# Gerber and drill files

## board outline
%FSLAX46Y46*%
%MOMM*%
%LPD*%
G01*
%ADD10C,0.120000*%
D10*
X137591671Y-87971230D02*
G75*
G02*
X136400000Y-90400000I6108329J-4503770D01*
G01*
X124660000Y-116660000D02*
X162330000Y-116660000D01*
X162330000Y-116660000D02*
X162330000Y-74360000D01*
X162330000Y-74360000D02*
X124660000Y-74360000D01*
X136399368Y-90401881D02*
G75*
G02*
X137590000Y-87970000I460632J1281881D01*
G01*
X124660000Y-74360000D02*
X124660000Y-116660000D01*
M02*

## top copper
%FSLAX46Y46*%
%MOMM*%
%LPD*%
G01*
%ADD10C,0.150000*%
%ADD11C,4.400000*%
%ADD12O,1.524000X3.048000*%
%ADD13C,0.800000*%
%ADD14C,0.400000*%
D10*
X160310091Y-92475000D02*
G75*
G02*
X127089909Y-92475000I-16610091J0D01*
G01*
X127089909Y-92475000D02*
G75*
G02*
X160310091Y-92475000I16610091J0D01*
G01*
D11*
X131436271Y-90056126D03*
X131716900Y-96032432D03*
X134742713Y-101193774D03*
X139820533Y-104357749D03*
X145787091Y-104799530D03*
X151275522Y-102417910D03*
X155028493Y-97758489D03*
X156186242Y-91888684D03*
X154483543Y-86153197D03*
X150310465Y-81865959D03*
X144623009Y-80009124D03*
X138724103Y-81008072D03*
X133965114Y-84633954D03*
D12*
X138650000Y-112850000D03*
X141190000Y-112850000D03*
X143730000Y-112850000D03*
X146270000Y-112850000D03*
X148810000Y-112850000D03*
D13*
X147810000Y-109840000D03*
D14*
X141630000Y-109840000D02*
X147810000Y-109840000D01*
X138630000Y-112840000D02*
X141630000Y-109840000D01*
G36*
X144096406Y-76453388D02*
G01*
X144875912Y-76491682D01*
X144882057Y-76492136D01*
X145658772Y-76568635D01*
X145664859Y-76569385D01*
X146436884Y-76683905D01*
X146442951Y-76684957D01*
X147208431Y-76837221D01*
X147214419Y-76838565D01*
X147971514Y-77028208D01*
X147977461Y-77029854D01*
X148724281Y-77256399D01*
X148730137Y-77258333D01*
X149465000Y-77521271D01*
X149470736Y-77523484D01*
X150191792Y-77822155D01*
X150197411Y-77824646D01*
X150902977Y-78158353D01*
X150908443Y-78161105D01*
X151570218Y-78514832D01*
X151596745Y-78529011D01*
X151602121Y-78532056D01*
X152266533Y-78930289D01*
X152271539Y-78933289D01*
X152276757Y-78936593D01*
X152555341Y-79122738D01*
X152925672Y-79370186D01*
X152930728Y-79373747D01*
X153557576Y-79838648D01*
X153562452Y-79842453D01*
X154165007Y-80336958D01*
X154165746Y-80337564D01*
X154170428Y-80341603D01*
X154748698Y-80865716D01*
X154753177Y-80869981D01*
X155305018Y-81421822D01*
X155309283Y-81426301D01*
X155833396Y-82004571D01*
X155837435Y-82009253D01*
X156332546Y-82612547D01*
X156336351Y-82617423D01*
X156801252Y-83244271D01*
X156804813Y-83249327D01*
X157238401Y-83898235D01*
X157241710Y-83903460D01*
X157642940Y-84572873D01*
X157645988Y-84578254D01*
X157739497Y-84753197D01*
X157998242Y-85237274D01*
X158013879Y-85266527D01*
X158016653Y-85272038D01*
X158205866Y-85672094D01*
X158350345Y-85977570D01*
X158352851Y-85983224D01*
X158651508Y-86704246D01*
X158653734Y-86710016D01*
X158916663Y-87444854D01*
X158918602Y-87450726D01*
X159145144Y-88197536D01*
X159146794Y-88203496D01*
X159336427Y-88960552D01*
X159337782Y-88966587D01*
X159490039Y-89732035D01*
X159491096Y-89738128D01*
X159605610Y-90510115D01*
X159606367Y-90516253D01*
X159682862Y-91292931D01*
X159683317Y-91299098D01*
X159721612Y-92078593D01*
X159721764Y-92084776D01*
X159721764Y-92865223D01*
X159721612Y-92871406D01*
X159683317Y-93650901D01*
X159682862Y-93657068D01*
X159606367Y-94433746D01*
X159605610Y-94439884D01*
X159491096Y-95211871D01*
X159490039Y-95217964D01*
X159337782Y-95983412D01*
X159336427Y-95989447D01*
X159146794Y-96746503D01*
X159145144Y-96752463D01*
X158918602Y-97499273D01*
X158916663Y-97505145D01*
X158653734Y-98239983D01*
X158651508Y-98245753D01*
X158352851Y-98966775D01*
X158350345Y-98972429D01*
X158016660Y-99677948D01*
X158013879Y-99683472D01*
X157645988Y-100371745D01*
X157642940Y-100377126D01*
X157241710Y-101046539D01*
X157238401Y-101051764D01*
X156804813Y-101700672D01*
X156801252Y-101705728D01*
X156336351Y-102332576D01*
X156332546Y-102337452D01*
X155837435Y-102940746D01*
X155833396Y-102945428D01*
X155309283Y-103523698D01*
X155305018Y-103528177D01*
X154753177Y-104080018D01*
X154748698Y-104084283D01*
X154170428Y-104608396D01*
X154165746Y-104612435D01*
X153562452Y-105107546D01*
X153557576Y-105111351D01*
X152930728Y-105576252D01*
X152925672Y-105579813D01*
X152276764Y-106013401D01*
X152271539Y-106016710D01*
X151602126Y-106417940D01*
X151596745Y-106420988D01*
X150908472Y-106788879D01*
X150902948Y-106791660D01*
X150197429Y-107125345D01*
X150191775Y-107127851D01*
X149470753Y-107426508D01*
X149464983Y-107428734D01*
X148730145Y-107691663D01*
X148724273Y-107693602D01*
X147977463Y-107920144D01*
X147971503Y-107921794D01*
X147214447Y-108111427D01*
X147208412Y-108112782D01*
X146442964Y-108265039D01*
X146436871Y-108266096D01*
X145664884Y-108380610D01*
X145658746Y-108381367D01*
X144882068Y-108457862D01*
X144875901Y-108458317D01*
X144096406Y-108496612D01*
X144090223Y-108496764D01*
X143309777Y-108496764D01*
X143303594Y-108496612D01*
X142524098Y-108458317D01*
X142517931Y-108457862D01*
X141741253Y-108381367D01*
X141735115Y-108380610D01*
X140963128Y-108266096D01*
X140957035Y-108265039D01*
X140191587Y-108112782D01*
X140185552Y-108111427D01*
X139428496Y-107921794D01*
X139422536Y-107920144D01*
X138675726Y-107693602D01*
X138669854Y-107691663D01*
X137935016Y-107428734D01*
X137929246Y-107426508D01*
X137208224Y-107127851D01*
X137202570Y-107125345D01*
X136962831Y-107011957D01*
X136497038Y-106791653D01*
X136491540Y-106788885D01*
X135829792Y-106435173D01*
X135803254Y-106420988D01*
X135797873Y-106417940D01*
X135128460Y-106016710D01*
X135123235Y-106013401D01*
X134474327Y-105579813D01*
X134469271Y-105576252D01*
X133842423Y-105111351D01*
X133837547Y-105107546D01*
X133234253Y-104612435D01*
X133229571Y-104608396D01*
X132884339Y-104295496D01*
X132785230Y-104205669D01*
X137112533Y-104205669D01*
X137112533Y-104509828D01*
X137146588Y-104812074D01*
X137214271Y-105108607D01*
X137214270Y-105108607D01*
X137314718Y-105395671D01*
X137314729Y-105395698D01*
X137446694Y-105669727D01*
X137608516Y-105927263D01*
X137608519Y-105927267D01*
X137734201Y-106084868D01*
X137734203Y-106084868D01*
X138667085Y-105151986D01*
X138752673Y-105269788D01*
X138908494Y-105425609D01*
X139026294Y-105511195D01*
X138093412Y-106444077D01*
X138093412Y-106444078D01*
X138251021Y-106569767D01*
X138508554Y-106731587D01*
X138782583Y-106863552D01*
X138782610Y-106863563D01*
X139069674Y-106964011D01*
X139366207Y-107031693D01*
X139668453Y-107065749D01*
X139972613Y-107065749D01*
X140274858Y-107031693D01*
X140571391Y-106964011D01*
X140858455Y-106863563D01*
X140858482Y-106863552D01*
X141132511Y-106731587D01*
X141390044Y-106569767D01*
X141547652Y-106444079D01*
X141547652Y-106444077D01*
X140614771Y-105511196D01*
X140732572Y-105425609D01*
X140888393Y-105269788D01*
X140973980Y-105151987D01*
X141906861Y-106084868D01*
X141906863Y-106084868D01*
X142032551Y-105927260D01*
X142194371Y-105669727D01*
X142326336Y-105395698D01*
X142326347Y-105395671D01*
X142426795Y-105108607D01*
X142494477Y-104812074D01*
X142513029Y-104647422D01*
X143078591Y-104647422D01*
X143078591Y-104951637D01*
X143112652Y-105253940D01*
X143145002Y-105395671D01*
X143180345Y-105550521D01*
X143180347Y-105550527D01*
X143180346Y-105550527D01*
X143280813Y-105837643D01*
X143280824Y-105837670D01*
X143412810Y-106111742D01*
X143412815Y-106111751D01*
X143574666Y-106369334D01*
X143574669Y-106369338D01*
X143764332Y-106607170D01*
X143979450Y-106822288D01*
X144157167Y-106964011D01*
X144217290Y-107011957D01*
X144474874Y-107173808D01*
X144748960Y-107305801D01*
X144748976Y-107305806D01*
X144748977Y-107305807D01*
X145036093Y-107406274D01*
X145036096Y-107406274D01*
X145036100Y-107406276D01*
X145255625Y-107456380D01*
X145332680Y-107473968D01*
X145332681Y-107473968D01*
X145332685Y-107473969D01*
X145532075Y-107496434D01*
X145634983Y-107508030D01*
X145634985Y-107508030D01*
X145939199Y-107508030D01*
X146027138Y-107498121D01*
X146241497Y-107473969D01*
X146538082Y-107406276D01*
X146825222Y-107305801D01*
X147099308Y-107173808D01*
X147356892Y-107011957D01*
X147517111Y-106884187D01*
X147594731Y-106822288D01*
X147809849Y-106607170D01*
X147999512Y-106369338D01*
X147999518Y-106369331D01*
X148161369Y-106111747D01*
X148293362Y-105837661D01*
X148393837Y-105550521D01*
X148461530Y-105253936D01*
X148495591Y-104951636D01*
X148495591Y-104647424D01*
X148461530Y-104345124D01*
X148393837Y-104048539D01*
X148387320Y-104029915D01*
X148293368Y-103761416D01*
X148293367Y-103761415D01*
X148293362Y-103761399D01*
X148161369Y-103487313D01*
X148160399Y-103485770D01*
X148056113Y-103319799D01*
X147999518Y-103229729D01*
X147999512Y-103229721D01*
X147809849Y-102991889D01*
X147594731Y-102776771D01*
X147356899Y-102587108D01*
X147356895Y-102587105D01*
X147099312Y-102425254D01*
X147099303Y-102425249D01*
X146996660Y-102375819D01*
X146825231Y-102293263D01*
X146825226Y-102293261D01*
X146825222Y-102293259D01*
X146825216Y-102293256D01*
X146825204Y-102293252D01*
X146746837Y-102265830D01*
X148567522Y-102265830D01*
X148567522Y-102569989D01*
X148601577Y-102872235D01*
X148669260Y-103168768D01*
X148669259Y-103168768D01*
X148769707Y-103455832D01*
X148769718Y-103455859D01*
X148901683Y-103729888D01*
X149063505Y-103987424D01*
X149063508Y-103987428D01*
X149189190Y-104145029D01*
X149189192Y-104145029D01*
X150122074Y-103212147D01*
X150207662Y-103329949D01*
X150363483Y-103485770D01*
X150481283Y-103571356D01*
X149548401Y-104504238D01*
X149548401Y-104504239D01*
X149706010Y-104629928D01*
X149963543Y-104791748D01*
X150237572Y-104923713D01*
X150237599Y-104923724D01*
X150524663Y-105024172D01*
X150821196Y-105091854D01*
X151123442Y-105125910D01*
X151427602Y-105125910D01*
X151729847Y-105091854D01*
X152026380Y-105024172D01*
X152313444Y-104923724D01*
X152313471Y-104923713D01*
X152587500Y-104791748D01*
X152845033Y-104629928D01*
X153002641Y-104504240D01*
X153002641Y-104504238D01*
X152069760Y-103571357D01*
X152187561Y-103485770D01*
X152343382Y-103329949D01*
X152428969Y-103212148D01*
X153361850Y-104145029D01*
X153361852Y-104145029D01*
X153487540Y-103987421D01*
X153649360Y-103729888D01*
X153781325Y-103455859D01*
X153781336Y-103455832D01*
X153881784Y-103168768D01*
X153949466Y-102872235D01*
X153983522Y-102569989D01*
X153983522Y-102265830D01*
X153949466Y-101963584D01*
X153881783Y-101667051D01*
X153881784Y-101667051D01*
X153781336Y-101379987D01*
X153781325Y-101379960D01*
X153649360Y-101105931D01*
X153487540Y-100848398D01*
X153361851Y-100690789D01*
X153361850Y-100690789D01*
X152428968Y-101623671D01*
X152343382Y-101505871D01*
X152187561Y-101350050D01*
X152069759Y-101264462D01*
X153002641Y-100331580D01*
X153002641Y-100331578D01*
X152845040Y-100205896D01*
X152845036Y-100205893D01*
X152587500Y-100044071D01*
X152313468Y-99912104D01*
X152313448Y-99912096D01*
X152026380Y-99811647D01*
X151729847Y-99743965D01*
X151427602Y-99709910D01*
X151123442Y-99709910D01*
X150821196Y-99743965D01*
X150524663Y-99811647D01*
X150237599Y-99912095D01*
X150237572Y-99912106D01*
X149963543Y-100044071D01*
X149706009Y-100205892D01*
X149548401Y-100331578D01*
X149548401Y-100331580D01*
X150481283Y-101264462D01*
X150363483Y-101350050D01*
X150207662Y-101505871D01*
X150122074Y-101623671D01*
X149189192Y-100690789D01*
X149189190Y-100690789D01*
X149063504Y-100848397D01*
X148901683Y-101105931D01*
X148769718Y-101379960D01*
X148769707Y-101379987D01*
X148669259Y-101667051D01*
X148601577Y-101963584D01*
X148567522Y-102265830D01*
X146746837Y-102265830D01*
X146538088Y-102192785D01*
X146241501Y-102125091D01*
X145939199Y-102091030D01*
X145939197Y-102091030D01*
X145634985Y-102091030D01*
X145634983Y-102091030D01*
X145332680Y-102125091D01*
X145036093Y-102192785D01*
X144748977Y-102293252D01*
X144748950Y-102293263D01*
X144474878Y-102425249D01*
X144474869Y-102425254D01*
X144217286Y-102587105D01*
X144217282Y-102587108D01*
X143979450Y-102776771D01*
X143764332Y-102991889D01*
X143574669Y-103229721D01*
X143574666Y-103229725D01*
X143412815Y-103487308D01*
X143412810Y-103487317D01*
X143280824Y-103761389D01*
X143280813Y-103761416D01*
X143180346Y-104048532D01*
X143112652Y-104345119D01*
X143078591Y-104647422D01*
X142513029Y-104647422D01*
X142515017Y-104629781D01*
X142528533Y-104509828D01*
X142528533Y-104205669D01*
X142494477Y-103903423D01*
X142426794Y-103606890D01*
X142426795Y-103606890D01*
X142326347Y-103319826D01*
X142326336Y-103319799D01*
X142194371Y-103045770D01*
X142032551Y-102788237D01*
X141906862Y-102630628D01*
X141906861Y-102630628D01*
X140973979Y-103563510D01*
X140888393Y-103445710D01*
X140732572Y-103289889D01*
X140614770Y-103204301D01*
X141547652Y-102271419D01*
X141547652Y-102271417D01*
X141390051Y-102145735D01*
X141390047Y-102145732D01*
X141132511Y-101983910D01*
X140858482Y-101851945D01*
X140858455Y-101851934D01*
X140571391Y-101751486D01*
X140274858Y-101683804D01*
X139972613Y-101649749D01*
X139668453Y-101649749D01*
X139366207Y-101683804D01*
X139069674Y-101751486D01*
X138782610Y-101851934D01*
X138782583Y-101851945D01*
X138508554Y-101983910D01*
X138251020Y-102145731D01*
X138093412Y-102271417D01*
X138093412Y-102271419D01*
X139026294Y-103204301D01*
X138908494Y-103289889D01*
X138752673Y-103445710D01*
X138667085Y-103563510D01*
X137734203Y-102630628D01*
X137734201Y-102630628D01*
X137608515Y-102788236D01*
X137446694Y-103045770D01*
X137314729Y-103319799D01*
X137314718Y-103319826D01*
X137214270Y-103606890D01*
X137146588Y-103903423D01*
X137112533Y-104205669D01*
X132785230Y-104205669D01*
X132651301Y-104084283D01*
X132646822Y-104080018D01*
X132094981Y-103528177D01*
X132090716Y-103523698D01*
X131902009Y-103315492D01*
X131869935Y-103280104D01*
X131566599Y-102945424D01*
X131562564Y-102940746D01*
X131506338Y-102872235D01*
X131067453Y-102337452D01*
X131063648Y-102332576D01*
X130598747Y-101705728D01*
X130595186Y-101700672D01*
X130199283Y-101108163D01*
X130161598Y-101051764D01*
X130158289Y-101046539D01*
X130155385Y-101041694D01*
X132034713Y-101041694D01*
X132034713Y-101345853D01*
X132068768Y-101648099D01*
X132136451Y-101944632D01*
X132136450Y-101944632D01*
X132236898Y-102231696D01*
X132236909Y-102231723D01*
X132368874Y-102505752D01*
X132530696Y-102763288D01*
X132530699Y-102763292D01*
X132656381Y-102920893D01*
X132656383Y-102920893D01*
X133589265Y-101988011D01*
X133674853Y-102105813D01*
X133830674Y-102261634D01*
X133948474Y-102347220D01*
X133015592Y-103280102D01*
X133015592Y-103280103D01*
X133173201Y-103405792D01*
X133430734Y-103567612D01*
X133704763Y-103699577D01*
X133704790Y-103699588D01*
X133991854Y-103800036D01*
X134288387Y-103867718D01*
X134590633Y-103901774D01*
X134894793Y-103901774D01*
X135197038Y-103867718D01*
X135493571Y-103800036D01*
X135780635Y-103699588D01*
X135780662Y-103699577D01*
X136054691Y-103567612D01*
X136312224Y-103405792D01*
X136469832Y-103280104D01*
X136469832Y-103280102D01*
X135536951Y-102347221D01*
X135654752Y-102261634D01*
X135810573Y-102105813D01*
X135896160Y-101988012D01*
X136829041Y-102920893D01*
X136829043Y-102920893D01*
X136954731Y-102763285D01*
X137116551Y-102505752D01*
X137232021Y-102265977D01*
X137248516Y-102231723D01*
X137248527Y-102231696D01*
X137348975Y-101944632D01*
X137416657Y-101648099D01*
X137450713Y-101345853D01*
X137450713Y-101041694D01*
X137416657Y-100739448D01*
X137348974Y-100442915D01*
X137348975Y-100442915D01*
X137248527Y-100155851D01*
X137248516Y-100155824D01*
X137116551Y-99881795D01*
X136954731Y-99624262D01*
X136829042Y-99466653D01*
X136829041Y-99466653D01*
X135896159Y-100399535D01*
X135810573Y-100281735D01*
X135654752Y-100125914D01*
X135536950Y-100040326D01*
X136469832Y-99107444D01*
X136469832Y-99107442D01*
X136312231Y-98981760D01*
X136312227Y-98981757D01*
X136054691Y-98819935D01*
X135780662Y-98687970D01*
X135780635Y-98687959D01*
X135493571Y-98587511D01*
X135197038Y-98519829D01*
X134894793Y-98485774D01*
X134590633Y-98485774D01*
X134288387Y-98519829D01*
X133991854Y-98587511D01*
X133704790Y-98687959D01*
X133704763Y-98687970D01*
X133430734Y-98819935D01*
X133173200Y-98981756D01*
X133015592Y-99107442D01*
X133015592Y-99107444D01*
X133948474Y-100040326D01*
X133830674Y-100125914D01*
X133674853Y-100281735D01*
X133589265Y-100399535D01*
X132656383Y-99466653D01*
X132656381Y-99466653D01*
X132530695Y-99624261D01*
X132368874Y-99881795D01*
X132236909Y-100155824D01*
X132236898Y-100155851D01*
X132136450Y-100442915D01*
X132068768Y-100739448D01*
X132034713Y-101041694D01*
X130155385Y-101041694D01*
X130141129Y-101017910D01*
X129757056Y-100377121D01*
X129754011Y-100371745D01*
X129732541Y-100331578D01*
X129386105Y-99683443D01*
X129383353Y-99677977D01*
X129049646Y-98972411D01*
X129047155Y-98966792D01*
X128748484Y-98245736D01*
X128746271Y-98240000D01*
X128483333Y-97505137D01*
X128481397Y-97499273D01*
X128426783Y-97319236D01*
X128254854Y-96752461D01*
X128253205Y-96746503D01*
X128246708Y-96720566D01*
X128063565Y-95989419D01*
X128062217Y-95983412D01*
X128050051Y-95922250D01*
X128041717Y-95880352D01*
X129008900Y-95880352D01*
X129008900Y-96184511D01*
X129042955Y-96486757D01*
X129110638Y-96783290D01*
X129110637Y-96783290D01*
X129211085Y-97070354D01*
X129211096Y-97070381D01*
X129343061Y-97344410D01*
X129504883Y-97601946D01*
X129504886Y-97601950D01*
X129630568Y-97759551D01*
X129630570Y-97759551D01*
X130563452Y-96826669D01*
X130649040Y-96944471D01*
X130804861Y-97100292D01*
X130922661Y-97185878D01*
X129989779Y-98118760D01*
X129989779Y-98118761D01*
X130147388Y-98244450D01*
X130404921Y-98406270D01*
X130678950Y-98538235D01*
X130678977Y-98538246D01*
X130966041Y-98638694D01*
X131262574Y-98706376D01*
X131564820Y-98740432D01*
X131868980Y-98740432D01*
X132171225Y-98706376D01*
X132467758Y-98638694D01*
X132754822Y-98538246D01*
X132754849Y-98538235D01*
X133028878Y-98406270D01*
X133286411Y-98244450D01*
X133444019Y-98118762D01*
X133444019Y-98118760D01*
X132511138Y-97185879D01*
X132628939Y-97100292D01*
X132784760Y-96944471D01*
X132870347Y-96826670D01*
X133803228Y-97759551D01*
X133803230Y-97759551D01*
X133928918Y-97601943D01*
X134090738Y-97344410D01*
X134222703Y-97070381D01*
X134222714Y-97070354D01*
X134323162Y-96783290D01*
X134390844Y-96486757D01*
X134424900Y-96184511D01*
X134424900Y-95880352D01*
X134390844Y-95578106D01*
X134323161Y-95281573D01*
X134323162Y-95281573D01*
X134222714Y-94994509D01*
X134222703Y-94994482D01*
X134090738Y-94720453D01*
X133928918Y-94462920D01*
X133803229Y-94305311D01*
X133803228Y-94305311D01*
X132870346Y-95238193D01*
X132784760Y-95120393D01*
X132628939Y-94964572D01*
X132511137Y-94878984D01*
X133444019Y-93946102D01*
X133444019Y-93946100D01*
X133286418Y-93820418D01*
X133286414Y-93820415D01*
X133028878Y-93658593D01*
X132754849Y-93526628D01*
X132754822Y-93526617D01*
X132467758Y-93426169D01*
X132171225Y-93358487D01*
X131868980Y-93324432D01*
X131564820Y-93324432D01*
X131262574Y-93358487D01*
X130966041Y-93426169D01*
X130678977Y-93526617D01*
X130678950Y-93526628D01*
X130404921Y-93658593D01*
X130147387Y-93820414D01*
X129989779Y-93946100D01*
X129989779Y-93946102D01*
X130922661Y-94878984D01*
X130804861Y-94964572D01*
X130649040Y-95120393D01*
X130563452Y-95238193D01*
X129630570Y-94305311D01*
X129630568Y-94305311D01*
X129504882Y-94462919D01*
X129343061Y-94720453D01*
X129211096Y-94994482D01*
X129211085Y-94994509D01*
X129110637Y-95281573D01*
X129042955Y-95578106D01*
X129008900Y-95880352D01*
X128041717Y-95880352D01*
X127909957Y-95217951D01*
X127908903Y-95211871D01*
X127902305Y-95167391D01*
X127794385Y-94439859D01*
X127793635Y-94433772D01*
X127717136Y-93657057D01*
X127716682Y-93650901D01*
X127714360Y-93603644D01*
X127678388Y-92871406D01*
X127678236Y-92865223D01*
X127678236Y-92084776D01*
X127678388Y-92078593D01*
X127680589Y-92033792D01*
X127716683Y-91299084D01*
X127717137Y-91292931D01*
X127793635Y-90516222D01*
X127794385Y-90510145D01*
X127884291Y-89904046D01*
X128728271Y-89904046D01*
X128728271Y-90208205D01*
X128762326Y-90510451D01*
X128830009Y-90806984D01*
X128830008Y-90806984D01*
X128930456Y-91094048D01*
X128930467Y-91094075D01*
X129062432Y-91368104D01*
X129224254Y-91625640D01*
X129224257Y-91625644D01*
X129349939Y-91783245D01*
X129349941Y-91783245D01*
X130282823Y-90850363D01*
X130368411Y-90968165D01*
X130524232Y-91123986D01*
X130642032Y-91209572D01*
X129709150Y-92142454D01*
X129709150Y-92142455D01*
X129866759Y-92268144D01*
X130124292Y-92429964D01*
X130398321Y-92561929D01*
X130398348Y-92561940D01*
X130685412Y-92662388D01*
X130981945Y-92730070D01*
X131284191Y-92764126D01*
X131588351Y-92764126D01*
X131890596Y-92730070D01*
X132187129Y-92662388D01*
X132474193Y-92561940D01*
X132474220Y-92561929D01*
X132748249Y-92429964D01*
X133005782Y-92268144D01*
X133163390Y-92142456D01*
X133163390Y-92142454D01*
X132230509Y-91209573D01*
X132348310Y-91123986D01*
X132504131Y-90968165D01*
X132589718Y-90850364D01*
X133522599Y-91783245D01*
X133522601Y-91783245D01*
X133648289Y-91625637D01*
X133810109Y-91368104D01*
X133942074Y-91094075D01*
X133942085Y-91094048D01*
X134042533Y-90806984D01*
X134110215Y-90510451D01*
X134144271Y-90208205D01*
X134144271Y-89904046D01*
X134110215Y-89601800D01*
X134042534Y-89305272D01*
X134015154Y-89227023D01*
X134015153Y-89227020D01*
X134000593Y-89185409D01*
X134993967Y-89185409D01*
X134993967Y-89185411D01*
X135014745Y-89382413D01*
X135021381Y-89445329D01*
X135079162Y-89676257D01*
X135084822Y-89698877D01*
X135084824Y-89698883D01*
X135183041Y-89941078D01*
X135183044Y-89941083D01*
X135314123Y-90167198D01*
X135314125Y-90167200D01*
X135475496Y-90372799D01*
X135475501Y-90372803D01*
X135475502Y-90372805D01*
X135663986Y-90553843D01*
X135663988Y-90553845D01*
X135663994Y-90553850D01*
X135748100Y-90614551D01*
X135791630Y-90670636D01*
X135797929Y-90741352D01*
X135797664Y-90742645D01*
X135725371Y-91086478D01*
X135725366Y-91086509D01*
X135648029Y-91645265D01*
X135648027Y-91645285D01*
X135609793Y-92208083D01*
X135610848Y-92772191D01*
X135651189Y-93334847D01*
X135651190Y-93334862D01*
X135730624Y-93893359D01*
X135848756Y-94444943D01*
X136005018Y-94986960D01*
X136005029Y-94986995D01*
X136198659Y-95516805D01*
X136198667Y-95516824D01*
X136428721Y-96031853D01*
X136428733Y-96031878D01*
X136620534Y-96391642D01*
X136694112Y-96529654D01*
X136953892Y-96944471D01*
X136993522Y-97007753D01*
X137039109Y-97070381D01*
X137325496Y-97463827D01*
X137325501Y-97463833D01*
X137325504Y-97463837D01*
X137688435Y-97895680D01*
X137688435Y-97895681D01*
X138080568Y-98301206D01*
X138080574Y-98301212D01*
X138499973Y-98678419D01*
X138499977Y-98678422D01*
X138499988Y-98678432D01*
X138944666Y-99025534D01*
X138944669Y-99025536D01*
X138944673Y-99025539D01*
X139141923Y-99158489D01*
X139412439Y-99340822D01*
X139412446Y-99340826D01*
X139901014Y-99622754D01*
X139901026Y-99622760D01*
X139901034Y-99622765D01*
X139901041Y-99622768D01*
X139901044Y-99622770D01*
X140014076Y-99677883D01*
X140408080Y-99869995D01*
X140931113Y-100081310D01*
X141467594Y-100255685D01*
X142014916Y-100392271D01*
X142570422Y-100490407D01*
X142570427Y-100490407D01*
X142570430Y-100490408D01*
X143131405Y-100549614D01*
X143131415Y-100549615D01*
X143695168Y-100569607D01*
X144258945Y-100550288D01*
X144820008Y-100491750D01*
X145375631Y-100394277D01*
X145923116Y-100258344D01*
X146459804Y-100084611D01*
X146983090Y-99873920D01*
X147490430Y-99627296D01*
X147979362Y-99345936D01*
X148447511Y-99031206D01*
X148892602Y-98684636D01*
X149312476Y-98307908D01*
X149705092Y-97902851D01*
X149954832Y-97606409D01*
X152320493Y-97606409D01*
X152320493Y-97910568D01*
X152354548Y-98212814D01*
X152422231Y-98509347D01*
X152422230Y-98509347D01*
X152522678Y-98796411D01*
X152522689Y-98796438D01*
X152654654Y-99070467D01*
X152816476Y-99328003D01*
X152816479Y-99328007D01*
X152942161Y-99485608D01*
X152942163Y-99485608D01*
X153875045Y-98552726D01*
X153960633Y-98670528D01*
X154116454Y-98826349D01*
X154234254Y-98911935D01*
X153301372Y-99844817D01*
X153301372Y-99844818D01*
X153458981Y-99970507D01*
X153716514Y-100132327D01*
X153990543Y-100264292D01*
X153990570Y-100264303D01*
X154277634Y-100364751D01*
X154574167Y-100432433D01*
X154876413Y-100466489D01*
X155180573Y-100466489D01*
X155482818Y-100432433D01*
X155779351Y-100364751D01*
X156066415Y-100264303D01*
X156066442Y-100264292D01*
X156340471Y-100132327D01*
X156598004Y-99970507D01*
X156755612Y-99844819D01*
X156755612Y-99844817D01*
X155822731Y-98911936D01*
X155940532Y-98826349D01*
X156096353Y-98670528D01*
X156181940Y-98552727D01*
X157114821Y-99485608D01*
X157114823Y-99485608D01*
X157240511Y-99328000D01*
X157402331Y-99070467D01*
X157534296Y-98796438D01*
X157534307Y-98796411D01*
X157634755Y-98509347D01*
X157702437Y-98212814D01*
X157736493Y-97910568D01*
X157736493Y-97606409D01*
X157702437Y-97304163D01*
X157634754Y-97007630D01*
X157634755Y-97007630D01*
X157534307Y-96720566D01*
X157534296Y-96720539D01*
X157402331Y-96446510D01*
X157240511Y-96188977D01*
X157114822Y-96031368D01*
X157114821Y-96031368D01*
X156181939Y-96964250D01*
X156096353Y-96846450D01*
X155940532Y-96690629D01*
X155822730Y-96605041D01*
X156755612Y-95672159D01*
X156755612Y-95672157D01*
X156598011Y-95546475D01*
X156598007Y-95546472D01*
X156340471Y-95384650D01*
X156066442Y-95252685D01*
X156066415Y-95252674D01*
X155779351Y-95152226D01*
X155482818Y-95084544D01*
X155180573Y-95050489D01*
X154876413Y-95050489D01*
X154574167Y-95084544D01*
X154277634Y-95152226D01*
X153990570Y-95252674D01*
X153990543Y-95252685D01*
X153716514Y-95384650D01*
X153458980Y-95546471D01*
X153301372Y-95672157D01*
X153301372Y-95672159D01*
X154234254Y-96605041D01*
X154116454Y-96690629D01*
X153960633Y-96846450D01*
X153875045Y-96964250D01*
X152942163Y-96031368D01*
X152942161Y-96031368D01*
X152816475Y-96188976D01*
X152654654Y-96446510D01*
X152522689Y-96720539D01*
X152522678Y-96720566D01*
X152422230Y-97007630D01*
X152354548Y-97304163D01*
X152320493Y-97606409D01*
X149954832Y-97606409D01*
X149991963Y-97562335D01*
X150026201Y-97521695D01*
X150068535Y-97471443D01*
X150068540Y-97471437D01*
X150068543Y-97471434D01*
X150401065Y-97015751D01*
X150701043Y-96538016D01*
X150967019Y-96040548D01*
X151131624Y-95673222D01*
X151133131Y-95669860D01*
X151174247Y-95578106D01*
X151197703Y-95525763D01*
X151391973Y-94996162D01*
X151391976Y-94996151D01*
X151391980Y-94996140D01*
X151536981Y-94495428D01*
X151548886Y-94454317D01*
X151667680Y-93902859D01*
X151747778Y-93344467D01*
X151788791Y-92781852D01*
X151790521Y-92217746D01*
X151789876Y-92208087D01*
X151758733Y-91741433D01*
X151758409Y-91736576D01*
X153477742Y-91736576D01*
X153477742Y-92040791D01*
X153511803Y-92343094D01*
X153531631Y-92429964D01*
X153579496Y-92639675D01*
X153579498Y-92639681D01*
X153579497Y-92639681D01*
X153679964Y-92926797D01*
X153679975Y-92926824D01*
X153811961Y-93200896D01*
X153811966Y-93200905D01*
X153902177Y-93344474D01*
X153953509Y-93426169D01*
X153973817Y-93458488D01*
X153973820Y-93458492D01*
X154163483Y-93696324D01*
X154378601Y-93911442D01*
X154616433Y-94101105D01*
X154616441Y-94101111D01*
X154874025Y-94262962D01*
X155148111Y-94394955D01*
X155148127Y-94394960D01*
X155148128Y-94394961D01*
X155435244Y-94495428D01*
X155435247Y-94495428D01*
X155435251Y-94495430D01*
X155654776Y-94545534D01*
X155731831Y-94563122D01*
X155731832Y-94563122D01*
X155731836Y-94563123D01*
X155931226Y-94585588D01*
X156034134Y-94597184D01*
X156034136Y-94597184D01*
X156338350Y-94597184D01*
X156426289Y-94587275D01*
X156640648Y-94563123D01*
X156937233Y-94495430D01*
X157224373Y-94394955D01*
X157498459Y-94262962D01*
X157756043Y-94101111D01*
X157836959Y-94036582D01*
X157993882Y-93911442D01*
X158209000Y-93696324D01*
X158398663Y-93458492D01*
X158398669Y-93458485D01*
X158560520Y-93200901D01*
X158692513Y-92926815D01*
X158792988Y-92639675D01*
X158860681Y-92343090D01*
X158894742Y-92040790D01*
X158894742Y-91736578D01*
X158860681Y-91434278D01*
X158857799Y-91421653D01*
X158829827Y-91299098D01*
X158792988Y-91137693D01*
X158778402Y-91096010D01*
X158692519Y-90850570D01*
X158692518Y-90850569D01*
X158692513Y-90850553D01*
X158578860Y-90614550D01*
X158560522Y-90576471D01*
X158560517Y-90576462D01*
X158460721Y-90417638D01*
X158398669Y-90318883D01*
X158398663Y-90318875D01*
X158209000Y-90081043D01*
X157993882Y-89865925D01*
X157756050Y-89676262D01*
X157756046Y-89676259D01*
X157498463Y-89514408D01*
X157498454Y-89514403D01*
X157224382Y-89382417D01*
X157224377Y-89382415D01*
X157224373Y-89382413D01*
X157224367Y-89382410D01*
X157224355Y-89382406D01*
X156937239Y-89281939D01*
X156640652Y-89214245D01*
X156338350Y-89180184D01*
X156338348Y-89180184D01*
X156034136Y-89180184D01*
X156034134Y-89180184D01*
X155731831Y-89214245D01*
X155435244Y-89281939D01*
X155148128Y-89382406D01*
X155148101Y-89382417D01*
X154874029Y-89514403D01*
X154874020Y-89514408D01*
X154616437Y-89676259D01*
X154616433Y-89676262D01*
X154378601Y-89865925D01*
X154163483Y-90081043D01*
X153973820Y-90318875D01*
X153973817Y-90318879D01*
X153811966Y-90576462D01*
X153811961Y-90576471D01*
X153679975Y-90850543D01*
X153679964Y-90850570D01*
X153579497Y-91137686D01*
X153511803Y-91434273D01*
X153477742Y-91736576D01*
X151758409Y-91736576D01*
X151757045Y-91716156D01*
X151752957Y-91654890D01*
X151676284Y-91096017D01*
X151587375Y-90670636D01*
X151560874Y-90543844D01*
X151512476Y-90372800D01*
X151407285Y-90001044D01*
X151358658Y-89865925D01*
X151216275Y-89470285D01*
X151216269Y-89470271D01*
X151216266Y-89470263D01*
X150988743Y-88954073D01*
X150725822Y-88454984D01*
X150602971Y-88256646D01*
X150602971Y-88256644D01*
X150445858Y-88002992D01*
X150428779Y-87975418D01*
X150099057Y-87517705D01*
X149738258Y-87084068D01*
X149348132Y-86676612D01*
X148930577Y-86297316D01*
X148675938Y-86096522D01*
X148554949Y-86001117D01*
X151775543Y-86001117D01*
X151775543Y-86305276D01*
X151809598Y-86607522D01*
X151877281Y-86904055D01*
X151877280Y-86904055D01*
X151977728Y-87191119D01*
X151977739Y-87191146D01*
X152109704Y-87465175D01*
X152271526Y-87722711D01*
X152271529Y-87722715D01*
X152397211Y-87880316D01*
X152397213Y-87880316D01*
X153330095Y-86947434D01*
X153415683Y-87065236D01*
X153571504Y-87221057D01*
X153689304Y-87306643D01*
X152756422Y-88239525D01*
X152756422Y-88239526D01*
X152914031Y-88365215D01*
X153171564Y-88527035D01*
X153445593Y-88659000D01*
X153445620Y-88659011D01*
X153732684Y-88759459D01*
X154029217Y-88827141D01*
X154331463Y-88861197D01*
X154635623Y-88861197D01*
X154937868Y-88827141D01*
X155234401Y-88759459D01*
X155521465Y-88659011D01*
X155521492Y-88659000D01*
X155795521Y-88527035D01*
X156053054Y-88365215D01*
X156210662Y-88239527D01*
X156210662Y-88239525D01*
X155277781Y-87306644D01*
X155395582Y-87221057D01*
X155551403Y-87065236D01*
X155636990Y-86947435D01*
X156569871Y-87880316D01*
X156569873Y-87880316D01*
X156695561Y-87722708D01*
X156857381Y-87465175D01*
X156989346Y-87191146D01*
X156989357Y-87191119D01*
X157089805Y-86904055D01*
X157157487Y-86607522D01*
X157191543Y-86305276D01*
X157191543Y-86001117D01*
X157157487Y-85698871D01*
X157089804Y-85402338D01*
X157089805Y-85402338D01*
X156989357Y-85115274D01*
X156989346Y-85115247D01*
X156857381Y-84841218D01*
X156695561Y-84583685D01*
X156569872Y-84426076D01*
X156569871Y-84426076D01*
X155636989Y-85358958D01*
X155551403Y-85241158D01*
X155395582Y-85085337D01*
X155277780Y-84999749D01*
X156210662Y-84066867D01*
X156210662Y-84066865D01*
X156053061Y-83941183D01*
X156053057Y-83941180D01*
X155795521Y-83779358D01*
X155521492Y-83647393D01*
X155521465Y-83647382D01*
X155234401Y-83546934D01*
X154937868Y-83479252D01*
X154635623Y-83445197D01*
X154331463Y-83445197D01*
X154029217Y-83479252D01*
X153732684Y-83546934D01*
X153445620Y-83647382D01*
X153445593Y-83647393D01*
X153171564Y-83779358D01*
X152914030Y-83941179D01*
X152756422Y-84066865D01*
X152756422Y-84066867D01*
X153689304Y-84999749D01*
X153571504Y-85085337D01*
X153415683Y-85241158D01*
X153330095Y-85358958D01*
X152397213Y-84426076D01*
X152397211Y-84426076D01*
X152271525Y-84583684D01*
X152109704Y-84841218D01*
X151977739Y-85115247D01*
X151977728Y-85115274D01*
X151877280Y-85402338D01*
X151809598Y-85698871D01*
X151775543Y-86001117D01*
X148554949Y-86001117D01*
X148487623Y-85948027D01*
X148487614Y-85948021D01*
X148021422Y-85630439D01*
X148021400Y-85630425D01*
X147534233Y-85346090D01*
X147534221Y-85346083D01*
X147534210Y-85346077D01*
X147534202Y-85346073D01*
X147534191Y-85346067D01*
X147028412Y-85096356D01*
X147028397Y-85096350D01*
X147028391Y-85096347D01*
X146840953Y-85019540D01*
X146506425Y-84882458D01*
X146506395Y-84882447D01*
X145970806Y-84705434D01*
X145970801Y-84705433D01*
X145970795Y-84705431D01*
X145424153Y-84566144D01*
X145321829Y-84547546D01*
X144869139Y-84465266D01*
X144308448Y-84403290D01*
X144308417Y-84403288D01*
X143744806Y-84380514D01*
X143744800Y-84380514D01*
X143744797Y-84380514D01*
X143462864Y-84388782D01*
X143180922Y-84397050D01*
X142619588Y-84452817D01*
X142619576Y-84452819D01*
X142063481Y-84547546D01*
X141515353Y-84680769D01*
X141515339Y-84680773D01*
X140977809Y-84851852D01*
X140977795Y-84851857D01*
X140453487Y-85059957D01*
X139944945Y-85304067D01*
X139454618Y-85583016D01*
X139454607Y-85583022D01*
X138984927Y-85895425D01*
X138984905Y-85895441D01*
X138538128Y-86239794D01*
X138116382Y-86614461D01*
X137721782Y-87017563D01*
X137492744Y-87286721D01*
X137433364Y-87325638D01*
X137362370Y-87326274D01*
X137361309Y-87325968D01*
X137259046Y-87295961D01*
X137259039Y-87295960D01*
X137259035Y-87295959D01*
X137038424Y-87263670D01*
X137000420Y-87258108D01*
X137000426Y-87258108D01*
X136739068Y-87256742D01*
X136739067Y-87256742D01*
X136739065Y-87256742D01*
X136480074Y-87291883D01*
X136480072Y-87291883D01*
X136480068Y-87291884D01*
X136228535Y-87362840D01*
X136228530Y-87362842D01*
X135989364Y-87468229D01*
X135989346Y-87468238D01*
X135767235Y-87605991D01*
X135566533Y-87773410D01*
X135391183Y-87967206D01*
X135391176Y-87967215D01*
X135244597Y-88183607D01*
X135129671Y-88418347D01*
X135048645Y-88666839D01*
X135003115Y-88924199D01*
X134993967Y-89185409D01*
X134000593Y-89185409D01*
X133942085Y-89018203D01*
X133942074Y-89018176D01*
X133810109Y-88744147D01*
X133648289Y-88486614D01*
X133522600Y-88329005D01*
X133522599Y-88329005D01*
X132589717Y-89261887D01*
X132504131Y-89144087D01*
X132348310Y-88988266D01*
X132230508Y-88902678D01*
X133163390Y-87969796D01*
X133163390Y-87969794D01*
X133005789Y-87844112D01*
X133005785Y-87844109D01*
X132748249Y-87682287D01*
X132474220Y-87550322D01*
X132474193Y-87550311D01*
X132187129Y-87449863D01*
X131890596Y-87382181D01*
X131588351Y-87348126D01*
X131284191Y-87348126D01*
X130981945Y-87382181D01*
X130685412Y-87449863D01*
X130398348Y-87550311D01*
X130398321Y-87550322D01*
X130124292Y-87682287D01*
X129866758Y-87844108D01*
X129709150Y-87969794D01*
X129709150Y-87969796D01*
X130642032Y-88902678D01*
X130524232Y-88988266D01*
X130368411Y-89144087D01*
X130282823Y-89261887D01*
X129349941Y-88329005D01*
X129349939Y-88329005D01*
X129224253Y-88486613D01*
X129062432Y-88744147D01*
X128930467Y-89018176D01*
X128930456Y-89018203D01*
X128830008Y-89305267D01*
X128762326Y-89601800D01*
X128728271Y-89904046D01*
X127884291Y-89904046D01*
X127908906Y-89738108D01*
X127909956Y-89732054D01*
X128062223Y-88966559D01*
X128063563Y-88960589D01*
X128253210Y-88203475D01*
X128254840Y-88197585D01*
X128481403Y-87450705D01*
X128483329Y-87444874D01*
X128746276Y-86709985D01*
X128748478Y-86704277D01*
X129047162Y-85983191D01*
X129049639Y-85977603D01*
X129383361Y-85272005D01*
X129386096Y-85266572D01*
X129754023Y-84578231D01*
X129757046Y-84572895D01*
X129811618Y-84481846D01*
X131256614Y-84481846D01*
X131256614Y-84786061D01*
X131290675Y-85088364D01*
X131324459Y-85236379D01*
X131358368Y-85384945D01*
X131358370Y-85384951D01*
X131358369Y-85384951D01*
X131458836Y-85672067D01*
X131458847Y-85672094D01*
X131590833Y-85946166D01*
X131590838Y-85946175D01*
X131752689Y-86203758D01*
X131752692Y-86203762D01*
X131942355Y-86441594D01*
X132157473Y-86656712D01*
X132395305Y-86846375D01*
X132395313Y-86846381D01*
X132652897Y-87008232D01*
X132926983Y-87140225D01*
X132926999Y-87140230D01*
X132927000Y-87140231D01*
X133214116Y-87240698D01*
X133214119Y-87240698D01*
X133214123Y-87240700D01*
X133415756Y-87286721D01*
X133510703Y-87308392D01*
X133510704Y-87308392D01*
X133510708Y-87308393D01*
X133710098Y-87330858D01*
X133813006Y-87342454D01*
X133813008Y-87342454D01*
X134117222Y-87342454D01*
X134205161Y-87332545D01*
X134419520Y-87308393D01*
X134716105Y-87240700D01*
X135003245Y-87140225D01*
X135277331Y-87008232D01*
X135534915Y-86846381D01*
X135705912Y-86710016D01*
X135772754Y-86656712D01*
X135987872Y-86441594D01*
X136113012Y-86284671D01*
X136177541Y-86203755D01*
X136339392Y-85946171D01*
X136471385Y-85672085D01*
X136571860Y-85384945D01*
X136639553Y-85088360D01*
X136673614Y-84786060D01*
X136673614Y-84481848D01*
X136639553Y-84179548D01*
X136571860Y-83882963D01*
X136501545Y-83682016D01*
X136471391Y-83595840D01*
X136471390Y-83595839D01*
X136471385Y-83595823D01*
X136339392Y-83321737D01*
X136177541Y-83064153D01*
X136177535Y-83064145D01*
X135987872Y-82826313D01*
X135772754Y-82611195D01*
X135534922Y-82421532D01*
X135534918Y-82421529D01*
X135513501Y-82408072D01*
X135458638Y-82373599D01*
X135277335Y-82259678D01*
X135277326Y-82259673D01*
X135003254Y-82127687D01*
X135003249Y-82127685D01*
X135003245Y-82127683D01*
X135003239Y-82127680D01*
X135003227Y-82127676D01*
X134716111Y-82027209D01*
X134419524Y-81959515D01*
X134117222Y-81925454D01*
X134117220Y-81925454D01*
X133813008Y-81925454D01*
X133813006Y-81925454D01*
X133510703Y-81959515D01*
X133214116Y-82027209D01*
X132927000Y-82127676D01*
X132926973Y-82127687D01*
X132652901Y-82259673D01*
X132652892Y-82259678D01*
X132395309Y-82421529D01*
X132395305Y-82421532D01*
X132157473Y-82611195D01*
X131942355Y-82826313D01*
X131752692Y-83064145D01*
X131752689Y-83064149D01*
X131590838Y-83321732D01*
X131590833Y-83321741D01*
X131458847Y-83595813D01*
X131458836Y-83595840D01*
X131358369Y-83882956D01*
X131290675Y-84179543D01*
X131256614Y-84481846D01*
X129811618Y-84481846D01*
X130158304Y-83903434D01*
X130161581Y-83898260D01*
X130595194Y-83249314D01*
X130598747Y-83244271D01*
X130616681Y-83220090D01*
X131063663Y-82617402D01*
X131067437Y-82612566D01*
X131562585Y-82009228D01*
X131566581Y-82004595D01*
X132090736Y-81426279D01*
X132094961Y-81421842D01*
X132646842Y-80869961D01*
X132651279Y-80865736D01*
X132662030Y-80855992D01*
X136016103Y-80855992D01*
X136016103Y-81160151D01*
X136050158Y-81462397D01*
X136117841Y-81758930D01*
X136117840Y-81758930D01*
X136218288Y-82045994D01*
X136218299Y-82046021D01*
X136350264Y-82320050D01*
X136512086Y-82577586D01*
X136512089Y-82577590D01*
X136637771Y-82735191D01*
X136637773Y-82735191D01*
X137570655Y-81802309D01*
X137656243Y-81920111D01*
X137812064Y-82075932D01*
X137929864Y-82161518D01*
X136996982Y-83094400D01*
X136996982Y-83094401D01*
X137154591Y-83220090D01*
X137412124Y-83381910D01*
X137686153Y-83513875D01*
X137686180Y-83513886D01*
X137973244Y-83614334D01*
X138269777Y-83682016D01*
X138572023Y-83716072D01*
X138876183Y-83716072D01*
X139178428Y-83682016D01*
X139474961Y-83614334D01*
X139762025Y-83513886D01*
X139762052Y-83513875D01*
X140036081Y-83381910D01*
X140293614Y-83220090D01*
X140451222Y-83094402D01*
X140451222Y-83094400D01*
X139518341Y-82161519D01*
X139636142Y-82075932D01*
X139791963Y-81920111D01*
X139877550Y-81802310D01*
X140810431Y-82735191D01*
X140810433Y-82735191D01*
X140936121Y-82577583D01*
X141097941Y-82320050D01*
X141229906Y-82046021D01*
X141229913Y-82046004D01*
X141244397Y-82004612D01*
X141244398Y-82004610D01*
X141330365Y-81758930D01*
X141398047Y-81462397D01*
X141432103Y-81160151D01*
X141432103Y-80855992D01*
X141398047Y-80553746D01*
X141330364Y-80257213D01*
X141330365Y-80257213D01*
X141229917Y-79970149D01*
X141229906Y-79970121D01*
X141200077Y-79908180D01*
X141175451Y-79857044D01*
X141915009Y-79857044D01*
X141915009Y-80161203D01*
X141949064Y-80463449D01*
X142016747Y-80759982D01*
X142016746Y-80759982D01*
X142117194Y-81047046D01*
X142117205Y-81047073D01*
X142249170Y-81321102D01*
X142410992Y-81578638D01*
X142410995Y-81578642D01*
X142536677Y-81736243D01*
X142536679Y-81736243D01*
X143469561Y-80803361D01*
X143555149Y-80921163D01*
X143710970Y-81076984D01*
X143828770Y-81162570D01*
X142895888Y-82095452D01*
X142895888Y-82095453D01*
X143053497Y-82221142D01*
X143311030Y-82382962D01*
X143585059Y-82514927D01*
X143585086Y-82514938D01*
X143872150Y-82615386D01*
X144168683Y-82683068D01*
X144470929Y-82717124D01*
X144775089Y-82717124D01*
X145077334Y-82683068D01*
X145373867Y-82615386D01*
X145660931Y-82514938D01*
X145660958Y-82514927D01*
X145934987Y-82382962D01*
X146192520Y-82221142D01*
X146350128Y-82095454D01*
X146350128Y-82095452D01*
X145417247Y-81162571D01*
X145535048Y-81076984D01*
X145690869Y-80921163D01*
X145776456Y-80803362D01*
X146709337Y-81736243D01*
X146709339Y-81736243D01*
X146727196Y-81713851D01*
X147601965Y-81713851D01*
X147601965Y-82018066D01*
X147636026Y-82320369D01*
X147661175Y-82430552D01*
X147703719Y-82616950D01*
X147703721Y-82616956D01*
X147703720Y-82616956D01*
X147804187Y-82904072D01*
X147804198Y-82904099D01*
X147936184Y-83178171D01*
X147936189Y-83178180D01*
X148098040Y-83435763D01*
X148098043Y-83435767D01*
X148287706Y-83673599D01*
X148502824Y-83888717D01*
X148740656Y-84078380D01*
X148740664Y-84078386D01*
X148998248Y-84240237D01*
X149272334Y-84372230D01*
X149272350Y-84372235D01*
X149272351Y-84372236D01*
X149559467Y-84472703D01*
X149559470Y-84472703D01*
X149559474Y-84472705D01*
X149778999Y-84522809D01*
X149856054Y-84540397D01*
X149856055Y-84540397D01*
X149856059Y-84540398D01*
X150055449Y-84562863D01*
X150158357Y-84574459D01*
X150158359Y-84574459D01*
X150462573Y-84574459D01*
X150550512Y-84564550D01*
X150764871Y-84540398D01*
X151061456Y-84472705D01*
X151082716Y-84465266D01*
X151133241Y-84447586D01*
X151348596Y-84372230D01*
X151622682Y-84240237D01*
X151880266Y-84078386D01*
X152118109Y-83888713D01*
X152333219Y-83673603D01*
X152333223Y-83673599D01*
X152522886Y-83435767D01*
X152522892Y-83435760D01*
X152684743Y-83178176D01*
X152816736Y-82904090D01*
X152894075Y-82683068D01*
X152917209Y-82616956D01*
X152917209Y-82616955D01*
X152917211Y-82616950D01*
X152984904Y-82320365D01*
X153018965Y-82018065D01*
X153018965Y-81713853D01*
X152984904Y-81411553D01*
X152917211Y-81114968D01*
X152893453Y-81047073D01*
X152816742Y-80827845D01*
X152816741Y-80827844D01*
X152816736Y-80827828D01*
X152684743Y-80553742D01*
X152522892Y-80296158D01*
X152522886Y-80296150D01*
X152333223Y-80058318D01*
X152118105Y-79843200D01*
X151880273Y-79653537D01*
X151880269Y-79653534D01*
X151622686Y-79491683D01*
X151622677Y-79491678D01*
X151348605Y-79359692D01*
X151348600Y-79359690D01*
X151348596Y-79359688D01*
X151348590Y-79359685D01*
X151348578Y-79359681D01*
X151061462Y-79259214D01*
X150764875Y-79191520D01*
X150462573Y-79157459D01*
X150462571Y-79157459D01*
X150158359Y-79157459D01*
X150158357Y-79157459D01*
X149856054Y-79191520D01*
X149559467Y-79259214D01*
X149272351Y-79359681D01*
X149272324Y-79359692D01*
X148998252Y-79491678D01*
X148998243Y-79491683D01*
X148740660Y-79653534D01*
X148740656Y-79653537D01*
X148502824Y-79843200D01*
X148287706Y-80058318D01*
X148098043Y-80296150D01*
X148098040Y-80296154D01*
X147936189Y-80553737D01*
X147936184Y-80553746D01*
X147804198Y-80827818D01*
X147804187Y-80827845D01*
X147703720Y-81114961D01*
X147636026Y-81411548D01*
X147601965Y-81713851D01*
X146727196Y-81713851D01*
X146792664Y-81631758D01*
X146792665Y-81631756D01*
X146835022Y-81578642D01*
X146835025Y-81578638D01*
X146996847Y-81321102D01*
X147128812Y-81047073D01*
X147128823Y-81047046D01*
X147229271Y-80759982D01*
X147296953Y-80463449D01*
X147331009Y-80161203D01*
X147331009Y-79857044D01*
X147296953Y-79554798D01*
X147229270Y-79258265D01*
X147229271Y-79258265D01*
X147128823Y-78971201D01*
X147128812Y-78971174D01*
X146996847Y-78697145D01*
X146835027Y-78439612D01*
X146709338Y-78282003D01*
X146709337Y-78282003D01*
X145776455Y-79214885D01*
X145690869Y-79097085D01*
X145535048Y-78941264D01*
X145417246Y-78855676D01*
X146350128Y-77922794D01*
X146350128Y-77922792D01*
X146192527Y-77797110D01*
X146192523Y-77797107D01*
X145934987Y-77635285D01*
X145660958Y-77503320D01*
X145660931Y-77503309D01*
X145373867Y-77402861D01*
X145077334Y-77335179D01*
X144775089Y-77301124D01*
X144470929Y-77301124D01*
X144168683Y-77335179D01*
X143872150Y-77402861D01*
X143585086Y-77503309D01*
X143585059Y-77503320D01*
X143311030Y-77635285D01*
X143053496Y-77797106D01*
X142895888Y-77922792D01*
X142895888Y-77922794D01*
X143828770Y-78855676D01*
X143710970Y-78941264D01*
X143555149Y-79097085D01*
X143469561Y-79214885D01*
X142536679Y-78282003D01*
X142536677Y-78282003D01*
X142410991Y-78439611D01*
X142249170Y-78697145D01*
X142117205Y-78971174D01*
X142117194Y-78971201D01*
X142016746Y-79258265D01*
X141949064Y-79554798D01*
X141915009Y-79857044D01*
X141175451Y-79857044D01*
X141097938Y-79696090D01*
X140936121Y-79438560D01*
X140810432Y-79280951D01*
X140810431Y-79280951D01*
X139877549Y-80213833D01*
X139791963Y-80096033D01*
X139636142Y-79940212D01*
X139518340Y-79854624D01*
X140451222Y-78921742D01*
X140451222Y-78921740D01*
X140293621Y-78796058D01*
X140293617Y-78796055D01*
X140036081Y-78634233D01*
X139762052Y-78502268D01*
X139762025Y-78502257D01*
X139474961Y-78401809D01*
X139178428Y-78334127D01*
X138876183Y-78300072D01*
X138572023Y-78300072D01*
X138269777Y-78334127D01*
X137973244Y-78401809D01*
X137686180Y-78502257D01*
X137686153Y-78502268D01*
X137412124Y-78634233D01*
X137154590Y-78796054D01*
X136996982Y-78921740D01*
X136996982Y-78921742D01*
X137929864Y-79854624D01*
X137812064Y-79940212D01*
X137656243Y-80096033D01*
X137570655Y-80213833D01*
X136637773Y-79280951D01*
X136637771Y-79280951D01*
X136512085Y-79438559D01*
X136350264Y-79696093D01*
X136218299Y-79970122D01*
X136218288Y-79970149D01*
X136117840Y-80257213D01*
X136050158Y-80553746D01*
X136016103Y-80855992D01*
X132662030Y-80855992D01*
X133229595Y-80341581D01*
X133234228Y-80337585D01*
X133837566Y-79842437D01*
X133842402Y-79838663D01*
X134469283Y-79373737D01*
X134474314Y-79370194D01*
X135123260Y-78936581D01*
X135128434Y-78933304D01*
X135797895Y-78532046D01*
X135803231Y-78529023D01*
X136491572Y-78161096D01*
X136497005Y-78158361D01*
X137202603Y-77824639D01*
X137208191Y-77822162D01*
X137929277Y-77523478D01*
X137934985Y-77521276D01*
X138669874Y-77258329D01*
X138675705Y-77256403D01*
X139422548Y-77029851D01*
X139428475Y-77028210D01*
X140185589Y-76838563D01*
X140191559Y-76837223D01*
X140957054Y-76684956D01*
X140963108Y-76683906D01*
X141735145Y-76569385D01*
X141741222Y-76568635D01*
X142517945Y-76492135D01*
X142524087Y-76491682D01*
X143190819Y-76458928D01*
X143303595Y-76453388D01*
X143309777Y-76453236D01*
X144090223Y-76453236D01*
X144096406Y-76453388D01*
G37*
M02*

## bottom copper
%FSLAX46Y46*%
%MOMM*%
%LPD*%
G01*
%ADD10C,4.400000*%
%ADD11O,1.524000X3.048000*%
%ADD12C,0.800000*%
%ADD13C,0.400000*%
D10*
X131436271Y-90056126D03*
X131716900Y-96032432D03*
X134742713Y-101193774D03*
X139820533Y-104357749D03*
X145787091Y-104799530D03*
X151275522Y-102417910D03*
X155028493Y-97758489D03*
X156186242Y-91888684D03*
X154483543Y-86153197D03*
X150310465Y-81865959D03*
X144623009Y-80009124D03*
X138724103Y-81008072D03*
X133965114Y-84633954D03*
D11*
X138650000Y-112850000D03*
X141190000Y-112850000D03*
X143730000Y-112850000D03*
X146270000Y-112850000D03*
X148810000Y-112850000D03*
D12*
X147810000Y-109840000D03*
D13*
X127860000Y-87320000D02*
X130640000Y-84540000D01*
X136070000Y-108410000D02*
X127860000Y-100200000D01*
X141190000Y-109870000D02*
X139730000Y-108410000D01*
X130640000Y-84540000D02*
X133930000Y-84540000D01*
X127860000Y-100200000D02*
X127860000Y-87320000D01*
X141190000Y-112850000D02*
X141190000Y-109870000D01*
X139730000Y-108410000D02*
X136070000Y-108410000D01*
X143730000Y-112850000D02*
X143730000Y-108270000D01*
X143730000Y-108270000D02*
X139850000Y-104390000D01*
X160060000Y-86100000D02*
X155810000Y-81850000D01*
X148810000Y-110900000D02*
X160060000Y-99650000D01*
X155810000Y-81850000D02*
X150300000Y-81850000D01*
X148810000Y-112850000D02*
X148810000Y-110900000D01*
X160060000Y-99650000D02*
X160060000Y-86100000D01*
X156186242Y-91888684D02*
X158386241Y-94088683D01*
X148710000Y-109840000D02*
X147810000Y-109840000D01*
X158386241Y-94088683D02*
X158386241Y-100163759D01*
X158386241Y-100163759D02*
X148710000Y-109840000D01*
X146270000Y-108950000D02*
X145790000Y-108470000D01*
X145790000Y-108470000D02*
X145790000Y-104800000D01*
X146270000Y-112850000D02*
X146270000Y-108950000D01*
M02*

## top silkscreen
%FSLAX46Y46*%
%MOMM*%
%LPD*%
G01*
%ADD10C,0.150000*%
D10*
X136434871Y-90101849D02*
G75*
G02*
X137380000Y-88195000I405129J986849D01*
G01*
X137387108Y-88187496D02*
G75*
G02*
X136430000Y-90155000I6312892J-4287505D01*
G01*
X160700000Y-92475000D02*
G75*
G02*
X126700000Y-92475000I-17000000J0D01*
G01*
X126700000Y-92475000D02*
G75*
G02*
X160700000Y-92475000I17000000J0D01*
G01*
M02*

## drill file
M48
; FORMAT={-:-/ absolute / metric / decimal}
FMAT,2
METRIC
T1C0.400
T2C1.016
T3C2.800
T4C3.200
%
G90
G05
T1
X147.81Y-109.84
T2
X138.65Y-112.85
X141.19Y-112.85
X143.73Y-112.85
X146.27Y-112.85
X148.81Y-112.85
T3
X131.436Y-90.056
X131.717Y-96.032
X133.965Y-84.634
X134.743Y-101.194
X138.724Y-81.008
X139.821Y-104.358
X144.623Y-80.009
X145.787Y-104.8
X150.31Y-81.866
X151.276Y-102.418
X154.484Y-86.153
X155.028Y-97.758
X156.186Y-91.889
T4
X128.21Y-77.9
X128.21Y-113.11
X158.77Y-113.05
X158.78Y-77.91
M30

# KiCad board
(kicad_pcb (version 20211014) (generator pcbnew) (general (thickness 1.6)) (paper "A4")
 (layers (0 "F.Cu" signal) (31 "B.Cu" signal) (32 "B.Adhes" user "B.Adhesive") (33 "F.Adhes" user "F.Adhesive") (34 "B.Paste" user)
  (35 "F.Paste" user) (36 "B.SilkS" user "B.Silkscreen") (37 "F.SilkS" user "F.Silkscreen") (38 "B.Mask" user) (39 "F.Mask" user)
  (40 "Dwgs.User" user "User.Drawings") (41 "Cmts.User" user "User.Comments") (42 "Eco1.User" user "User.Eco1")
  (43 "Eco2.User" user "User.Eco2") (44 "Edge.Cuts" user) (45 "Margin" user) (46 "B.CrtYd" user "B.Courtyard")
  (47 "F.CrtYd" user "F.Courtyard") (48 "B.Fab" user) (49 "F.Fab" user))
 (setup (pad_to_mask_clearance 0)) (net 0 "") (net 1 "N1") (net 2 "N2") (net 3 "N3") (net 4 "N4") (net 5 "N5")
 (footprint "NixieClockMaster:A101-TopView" (layer "F.Cu") (at 143.7 92.475)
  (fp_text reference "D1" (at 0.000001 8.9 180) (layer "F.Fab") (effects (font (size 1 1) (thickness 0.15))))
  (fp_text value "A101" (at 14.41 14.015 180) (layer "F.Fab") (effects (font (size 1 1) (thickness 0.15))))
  (fp_arc (start -7.265129 -2.373151) (mid -7.815806 -3.833745) (end -6.32 -4.28) (layer "F.SilkS") (width 0.15))
  (fp_arc (start -6.312892 -4.287504) (mid 6.862325 3.338232) (end -7.27 -2.32) (layer "F.SilkS") (width 0.15))
  (fp_circle (center 0 0) (end 17 0) (layer "F.SilkS") (width 0.15) (fill none))
  (pad "1" thru_hole circle locked (at -12.263729 -2.418874) (size 4.4 4.4) (drill 2.8) (layers *.Cu *.Mask) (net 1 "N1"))
  (pad "2" thru_hole circle locked (at -11.9831 3.557432) (size 4.4 4.4) (drill 2.8) (layers *.Cu *.Mask) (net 1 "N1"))
  (pad "3" thru_hole circle locked (at -8.957287 8.718774) (size 4.4 4.4) (drill 2.8) (layers *.Cu *.Mask) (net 1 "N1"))
  (pad "4" thru_hole circle locked (at -3.879467 11.882749) (size 4.4 4.4) (drill 2.8) (layers *.Cu *.Mask) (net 1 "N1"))
  (pad "5" thru_hole circle locked (at 2.087091 12.32453) (size 4.4 4.4) (drill 2.8) (layers *.Cu *.Mask) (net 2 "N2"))
  (pad "6" thru_hole circle locked (at 7.575522 9.94291) (size 4.4 4.4) (drill 2.8) (layers *.Cu *.Mask) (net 1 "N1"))
  (pad "7" thru_hole circle locked (at 11.328493 5.283489) (size 4.4 4.4) (drill 2.8) (layers *.Cu *.Mask) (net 1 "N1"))
  (pad "8" thru_hole circle locked (at 12.486242 -0.586316) (size 4.4 4.4) (drill 2.8) (layers *.Cu *.Mask) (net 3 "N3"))
  (pad "9" thru_hole circle locked (at 10.783543 -6.321803) (size 4.4 4.4) (drill 2.8) (layers *.Cu *.Mask) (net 1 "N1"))
  (pad "10" thru_hole circle locked (at 6.610465 -10.609041) (size 4.4 4.4) (drill 2.8) (layers *.Cu *.Mask) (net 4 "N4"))
  (pad "11" thru_hole circle locked (at 0.923009 -12.465876) (size 4.4 4.4) (drill 2.8) (layers *.Cu *.Mask) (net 1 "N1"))
  (pad "12" thru_hole circle locked (at -4.975897 -11.466928) (size 4.4 4.4) (drill 2.8) (layers *.Cu *.Mask) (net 1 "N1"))
  (pad "13" thru_hole circle locked (at -9.734886 -7.841046) (size 4.4 4.4) (drill 2.8) (layers *.Cu *.Mask) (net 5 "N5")))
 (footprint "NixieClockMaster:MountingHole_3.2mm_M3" (layer "F.Cu") (at 128.21 77.9)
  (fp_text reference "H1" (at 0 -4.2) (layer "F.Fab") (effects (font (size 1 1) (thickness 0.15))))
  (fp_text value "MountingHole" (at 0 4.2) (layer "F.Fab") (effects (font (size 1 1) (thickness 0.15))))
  (pad "" np_thru_hole circle locked (at 0 0) (size 3.2 3.2) (drill 3.2) (layers *.Cu *.Mask)))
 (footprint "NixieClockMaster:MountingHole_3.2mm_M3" (layer "F.Cu") (at 128.21 113.11)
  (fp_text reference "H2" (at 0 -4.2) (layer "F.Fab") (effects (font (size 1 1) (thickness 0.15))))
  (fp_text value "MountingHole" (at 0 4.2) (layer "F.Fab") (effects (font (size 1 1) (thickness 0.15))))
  (pad "" np_thru_hole circle locked (at 0 0) (size 3.2 3.2) (drill 3.2) (layers *.Cu *.Mask)))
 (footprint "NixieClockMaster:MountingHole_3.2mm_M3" (layer "F.Cu") (at 158.78 77.91)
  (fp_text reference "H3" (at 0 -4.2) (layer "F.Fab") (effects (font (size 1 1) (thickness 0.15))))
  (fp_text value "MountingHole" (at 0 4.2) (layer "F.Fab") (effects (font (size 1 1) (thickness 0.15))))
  (pad "" np_thru_hole circle locked (at 0 0) (size 3.2 3.2) (drill 3.2) (layers *.Cu *.Mask)))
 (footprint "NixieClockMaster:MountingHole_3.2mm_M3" (layer "F.Cu") (at 158.77 113.05)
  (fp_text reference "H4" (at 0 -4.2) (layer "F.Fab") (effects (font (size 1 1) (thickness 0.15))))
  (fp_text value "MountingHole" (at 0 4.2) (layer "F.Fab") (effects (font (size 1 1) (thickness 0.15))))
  (pad "" np_thru_hole circle locked (at 0 0) (size 3.2 3.2) (drill 3.2) (layers *.Cu *.Mask)))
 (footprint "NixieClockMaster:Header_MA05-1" (layer "B.Cu") (at 145 112.85)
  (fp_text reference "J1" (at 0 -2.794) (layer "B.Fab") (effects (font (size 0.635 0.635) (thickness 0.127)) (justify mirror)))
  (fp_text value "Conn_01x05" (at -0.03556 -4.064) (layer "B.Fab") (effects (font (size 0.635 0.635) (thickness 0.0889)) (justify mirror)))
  (pad "1" thru_hole oval (at -6.35 0 180) (size 1.524 3.048) (drill 1.016) (layers *.Cu *.Mask) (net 3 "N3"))
  (pad "2" thru_hole oval (at -3.81 0 180) (size 1.524 3.048) (drill 1.016) (layers *.Cu *.Mask) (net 5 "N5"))
  (pad "3" thru_hole oval (at -1.27 0 180) (size 1.524 3.048) (drill 1.016) (layers *.Cu *.Mask) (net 1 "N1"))
  (pad "4" thru_hole oval (at 1.27 0 180) (size 1.524 3.048) (drill 1.016) (layers *.Cu *.Mask) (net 2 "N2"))
  (pad "5" thru_hole oval (at 3.81 0 180) (size 1.524 3.048) (drill 1.016) (layers *.Cu *.Mask) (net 4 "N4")))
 (gr_circle (center 143.7 92.475) (end 160.310091 92.475) (layer "F.Cu") (width 0.15) (fill none))
 (gr_arc (start 137.591671 87.97123) (mid 150.513263 95.817914) (end 136.4 90.4) (layer "Edge.Cuts") (width 0.12))
 (gr_line (start 124.66 116.66) (end 162.33 116.66) (layer "Edge.Cuts") (width 0.12))
 (gr_line (start 162.33 116.66) (end 162.33 74.36) (layer "Edge.Cuts") (width 0.12))
 (gr_line (start 162.33 74.36) (end 124.66 74.36) (layer "Edge.Cuts") (width 0.12))
 (gr_arc (start 136.399368 90.401881) (mid 135.636623 88.521043) (end 137.59 87.97) (layer "Edge.Cuts") (width 0.12))
 (gr_line (start 124.66 74.36) (end 124.66 116.66) (layer "Edge.Cuts") (width 0.12))
 (segment (start 127.86 87.32) (end 130.64 84.54) (width 0.4) (layer "B.Cu") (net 5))
 (segment (start 136.07 108.41) (end 127.86 100.2) (width 0.4) (layer "B.Cu") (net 5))
 (segment (start 141.19 109.87) (end 139.73 108.41) (width 0.4) (layer "B.Cu") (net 5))
 (segment (start 130.64 84.54) (end 133.93 84.54) (width 0.4) (layer "B.Cu") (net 5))
 (segment (start 127.86 100.2) (end 127.86 87.32) (width 0.4) (layer "B.Cu") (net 5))
 (segment (start 141.19 112.85) (end 141.19 109.87) (width 0.4) (layer "B.Cu") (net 5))
 (segment (start 139.73 108.41) (end 136.07 108.41) (width 0.4) (layer "B.Cu") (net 5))
 (segment (start 143.73 112.85) (end 143.73 108.27) (width 0.4) (layer "B.Cu") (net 1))
 (segment (start 143.73 108.27) (end 139.85 104.39) (width 0.4) (layer "B.Cu") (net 1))
 (segment (start 160.06 86.1) (end 155.81 81.85) (width 0.4) (layer "B.Cu") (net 4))
 (segment (start 148.81 110.9) (end 160.06 99.65) (width 0.4) (layer "B.Cu") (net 4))
 (segment (start 155.81 81.85) (end 150.3 81.85) (width 0.4) (layer "B.Cu") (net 4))
 (segment (start 148.81 112.85) (end 148.81 110.9) (width 0.4) (layer "B.Cu") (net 4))
 (segment (start 160.06 99.65) (end 160.06 86.1) (width 0.4) (layer "B.Cu") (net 4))
 (segment (start 141.63 109.84) (end 147.81 109.84) (width 0.4) (layer "F.Cu") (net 3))
 (segment (start 138.63 112.84) (end 141.63 109.84) (width 0.4) (layer "F.Cu") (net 3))
 (via (at 147.81 109.84) (size 0.8) (drill 0.4) (layers "F.Cu" "B.Cu") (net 3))
 (segment (start 156.186242 91.888684) (end 158.386241 94.088683) (width 0.4) (layer "B.Cu") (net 3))
 (segment (start 148.71 109.84) (end 147.81 109.84) (width 0.4) (layer "B.Cu") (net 3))
 (segment (start 158.386241 94.088683) (end 158.386241 100.163759) (width 0.4) (layer "B.Cu") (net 3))
 (segment (start 158.386241 100.163759) (end 148.71 109.84) (width 0.4) (layer "B.Cu") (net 3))
 (segment (start 146.27 108.95) (end 145.79 108.47) (width 0.4) (layer "B.Cu") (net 2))
 (segment (start 145.79 108.47) (end 145.79 104.8) (width 0.4) (layer "B.Cu") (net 2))
 (segment (start 146.27 112.85) (end 146.27 108.95) (width 0.4) (layer "B.Cu") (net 2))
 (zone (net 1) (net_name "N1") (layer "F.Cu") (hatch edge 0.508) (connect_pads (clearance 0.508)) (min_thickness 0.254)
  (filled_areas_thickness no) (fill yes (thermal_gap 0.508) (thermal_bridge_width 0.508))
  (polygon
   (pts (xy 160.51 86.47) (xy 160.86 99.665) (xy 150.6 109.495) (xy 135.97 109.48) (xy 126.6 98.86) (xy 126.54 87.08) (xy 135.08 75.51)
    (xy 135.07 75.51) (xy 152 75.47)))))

